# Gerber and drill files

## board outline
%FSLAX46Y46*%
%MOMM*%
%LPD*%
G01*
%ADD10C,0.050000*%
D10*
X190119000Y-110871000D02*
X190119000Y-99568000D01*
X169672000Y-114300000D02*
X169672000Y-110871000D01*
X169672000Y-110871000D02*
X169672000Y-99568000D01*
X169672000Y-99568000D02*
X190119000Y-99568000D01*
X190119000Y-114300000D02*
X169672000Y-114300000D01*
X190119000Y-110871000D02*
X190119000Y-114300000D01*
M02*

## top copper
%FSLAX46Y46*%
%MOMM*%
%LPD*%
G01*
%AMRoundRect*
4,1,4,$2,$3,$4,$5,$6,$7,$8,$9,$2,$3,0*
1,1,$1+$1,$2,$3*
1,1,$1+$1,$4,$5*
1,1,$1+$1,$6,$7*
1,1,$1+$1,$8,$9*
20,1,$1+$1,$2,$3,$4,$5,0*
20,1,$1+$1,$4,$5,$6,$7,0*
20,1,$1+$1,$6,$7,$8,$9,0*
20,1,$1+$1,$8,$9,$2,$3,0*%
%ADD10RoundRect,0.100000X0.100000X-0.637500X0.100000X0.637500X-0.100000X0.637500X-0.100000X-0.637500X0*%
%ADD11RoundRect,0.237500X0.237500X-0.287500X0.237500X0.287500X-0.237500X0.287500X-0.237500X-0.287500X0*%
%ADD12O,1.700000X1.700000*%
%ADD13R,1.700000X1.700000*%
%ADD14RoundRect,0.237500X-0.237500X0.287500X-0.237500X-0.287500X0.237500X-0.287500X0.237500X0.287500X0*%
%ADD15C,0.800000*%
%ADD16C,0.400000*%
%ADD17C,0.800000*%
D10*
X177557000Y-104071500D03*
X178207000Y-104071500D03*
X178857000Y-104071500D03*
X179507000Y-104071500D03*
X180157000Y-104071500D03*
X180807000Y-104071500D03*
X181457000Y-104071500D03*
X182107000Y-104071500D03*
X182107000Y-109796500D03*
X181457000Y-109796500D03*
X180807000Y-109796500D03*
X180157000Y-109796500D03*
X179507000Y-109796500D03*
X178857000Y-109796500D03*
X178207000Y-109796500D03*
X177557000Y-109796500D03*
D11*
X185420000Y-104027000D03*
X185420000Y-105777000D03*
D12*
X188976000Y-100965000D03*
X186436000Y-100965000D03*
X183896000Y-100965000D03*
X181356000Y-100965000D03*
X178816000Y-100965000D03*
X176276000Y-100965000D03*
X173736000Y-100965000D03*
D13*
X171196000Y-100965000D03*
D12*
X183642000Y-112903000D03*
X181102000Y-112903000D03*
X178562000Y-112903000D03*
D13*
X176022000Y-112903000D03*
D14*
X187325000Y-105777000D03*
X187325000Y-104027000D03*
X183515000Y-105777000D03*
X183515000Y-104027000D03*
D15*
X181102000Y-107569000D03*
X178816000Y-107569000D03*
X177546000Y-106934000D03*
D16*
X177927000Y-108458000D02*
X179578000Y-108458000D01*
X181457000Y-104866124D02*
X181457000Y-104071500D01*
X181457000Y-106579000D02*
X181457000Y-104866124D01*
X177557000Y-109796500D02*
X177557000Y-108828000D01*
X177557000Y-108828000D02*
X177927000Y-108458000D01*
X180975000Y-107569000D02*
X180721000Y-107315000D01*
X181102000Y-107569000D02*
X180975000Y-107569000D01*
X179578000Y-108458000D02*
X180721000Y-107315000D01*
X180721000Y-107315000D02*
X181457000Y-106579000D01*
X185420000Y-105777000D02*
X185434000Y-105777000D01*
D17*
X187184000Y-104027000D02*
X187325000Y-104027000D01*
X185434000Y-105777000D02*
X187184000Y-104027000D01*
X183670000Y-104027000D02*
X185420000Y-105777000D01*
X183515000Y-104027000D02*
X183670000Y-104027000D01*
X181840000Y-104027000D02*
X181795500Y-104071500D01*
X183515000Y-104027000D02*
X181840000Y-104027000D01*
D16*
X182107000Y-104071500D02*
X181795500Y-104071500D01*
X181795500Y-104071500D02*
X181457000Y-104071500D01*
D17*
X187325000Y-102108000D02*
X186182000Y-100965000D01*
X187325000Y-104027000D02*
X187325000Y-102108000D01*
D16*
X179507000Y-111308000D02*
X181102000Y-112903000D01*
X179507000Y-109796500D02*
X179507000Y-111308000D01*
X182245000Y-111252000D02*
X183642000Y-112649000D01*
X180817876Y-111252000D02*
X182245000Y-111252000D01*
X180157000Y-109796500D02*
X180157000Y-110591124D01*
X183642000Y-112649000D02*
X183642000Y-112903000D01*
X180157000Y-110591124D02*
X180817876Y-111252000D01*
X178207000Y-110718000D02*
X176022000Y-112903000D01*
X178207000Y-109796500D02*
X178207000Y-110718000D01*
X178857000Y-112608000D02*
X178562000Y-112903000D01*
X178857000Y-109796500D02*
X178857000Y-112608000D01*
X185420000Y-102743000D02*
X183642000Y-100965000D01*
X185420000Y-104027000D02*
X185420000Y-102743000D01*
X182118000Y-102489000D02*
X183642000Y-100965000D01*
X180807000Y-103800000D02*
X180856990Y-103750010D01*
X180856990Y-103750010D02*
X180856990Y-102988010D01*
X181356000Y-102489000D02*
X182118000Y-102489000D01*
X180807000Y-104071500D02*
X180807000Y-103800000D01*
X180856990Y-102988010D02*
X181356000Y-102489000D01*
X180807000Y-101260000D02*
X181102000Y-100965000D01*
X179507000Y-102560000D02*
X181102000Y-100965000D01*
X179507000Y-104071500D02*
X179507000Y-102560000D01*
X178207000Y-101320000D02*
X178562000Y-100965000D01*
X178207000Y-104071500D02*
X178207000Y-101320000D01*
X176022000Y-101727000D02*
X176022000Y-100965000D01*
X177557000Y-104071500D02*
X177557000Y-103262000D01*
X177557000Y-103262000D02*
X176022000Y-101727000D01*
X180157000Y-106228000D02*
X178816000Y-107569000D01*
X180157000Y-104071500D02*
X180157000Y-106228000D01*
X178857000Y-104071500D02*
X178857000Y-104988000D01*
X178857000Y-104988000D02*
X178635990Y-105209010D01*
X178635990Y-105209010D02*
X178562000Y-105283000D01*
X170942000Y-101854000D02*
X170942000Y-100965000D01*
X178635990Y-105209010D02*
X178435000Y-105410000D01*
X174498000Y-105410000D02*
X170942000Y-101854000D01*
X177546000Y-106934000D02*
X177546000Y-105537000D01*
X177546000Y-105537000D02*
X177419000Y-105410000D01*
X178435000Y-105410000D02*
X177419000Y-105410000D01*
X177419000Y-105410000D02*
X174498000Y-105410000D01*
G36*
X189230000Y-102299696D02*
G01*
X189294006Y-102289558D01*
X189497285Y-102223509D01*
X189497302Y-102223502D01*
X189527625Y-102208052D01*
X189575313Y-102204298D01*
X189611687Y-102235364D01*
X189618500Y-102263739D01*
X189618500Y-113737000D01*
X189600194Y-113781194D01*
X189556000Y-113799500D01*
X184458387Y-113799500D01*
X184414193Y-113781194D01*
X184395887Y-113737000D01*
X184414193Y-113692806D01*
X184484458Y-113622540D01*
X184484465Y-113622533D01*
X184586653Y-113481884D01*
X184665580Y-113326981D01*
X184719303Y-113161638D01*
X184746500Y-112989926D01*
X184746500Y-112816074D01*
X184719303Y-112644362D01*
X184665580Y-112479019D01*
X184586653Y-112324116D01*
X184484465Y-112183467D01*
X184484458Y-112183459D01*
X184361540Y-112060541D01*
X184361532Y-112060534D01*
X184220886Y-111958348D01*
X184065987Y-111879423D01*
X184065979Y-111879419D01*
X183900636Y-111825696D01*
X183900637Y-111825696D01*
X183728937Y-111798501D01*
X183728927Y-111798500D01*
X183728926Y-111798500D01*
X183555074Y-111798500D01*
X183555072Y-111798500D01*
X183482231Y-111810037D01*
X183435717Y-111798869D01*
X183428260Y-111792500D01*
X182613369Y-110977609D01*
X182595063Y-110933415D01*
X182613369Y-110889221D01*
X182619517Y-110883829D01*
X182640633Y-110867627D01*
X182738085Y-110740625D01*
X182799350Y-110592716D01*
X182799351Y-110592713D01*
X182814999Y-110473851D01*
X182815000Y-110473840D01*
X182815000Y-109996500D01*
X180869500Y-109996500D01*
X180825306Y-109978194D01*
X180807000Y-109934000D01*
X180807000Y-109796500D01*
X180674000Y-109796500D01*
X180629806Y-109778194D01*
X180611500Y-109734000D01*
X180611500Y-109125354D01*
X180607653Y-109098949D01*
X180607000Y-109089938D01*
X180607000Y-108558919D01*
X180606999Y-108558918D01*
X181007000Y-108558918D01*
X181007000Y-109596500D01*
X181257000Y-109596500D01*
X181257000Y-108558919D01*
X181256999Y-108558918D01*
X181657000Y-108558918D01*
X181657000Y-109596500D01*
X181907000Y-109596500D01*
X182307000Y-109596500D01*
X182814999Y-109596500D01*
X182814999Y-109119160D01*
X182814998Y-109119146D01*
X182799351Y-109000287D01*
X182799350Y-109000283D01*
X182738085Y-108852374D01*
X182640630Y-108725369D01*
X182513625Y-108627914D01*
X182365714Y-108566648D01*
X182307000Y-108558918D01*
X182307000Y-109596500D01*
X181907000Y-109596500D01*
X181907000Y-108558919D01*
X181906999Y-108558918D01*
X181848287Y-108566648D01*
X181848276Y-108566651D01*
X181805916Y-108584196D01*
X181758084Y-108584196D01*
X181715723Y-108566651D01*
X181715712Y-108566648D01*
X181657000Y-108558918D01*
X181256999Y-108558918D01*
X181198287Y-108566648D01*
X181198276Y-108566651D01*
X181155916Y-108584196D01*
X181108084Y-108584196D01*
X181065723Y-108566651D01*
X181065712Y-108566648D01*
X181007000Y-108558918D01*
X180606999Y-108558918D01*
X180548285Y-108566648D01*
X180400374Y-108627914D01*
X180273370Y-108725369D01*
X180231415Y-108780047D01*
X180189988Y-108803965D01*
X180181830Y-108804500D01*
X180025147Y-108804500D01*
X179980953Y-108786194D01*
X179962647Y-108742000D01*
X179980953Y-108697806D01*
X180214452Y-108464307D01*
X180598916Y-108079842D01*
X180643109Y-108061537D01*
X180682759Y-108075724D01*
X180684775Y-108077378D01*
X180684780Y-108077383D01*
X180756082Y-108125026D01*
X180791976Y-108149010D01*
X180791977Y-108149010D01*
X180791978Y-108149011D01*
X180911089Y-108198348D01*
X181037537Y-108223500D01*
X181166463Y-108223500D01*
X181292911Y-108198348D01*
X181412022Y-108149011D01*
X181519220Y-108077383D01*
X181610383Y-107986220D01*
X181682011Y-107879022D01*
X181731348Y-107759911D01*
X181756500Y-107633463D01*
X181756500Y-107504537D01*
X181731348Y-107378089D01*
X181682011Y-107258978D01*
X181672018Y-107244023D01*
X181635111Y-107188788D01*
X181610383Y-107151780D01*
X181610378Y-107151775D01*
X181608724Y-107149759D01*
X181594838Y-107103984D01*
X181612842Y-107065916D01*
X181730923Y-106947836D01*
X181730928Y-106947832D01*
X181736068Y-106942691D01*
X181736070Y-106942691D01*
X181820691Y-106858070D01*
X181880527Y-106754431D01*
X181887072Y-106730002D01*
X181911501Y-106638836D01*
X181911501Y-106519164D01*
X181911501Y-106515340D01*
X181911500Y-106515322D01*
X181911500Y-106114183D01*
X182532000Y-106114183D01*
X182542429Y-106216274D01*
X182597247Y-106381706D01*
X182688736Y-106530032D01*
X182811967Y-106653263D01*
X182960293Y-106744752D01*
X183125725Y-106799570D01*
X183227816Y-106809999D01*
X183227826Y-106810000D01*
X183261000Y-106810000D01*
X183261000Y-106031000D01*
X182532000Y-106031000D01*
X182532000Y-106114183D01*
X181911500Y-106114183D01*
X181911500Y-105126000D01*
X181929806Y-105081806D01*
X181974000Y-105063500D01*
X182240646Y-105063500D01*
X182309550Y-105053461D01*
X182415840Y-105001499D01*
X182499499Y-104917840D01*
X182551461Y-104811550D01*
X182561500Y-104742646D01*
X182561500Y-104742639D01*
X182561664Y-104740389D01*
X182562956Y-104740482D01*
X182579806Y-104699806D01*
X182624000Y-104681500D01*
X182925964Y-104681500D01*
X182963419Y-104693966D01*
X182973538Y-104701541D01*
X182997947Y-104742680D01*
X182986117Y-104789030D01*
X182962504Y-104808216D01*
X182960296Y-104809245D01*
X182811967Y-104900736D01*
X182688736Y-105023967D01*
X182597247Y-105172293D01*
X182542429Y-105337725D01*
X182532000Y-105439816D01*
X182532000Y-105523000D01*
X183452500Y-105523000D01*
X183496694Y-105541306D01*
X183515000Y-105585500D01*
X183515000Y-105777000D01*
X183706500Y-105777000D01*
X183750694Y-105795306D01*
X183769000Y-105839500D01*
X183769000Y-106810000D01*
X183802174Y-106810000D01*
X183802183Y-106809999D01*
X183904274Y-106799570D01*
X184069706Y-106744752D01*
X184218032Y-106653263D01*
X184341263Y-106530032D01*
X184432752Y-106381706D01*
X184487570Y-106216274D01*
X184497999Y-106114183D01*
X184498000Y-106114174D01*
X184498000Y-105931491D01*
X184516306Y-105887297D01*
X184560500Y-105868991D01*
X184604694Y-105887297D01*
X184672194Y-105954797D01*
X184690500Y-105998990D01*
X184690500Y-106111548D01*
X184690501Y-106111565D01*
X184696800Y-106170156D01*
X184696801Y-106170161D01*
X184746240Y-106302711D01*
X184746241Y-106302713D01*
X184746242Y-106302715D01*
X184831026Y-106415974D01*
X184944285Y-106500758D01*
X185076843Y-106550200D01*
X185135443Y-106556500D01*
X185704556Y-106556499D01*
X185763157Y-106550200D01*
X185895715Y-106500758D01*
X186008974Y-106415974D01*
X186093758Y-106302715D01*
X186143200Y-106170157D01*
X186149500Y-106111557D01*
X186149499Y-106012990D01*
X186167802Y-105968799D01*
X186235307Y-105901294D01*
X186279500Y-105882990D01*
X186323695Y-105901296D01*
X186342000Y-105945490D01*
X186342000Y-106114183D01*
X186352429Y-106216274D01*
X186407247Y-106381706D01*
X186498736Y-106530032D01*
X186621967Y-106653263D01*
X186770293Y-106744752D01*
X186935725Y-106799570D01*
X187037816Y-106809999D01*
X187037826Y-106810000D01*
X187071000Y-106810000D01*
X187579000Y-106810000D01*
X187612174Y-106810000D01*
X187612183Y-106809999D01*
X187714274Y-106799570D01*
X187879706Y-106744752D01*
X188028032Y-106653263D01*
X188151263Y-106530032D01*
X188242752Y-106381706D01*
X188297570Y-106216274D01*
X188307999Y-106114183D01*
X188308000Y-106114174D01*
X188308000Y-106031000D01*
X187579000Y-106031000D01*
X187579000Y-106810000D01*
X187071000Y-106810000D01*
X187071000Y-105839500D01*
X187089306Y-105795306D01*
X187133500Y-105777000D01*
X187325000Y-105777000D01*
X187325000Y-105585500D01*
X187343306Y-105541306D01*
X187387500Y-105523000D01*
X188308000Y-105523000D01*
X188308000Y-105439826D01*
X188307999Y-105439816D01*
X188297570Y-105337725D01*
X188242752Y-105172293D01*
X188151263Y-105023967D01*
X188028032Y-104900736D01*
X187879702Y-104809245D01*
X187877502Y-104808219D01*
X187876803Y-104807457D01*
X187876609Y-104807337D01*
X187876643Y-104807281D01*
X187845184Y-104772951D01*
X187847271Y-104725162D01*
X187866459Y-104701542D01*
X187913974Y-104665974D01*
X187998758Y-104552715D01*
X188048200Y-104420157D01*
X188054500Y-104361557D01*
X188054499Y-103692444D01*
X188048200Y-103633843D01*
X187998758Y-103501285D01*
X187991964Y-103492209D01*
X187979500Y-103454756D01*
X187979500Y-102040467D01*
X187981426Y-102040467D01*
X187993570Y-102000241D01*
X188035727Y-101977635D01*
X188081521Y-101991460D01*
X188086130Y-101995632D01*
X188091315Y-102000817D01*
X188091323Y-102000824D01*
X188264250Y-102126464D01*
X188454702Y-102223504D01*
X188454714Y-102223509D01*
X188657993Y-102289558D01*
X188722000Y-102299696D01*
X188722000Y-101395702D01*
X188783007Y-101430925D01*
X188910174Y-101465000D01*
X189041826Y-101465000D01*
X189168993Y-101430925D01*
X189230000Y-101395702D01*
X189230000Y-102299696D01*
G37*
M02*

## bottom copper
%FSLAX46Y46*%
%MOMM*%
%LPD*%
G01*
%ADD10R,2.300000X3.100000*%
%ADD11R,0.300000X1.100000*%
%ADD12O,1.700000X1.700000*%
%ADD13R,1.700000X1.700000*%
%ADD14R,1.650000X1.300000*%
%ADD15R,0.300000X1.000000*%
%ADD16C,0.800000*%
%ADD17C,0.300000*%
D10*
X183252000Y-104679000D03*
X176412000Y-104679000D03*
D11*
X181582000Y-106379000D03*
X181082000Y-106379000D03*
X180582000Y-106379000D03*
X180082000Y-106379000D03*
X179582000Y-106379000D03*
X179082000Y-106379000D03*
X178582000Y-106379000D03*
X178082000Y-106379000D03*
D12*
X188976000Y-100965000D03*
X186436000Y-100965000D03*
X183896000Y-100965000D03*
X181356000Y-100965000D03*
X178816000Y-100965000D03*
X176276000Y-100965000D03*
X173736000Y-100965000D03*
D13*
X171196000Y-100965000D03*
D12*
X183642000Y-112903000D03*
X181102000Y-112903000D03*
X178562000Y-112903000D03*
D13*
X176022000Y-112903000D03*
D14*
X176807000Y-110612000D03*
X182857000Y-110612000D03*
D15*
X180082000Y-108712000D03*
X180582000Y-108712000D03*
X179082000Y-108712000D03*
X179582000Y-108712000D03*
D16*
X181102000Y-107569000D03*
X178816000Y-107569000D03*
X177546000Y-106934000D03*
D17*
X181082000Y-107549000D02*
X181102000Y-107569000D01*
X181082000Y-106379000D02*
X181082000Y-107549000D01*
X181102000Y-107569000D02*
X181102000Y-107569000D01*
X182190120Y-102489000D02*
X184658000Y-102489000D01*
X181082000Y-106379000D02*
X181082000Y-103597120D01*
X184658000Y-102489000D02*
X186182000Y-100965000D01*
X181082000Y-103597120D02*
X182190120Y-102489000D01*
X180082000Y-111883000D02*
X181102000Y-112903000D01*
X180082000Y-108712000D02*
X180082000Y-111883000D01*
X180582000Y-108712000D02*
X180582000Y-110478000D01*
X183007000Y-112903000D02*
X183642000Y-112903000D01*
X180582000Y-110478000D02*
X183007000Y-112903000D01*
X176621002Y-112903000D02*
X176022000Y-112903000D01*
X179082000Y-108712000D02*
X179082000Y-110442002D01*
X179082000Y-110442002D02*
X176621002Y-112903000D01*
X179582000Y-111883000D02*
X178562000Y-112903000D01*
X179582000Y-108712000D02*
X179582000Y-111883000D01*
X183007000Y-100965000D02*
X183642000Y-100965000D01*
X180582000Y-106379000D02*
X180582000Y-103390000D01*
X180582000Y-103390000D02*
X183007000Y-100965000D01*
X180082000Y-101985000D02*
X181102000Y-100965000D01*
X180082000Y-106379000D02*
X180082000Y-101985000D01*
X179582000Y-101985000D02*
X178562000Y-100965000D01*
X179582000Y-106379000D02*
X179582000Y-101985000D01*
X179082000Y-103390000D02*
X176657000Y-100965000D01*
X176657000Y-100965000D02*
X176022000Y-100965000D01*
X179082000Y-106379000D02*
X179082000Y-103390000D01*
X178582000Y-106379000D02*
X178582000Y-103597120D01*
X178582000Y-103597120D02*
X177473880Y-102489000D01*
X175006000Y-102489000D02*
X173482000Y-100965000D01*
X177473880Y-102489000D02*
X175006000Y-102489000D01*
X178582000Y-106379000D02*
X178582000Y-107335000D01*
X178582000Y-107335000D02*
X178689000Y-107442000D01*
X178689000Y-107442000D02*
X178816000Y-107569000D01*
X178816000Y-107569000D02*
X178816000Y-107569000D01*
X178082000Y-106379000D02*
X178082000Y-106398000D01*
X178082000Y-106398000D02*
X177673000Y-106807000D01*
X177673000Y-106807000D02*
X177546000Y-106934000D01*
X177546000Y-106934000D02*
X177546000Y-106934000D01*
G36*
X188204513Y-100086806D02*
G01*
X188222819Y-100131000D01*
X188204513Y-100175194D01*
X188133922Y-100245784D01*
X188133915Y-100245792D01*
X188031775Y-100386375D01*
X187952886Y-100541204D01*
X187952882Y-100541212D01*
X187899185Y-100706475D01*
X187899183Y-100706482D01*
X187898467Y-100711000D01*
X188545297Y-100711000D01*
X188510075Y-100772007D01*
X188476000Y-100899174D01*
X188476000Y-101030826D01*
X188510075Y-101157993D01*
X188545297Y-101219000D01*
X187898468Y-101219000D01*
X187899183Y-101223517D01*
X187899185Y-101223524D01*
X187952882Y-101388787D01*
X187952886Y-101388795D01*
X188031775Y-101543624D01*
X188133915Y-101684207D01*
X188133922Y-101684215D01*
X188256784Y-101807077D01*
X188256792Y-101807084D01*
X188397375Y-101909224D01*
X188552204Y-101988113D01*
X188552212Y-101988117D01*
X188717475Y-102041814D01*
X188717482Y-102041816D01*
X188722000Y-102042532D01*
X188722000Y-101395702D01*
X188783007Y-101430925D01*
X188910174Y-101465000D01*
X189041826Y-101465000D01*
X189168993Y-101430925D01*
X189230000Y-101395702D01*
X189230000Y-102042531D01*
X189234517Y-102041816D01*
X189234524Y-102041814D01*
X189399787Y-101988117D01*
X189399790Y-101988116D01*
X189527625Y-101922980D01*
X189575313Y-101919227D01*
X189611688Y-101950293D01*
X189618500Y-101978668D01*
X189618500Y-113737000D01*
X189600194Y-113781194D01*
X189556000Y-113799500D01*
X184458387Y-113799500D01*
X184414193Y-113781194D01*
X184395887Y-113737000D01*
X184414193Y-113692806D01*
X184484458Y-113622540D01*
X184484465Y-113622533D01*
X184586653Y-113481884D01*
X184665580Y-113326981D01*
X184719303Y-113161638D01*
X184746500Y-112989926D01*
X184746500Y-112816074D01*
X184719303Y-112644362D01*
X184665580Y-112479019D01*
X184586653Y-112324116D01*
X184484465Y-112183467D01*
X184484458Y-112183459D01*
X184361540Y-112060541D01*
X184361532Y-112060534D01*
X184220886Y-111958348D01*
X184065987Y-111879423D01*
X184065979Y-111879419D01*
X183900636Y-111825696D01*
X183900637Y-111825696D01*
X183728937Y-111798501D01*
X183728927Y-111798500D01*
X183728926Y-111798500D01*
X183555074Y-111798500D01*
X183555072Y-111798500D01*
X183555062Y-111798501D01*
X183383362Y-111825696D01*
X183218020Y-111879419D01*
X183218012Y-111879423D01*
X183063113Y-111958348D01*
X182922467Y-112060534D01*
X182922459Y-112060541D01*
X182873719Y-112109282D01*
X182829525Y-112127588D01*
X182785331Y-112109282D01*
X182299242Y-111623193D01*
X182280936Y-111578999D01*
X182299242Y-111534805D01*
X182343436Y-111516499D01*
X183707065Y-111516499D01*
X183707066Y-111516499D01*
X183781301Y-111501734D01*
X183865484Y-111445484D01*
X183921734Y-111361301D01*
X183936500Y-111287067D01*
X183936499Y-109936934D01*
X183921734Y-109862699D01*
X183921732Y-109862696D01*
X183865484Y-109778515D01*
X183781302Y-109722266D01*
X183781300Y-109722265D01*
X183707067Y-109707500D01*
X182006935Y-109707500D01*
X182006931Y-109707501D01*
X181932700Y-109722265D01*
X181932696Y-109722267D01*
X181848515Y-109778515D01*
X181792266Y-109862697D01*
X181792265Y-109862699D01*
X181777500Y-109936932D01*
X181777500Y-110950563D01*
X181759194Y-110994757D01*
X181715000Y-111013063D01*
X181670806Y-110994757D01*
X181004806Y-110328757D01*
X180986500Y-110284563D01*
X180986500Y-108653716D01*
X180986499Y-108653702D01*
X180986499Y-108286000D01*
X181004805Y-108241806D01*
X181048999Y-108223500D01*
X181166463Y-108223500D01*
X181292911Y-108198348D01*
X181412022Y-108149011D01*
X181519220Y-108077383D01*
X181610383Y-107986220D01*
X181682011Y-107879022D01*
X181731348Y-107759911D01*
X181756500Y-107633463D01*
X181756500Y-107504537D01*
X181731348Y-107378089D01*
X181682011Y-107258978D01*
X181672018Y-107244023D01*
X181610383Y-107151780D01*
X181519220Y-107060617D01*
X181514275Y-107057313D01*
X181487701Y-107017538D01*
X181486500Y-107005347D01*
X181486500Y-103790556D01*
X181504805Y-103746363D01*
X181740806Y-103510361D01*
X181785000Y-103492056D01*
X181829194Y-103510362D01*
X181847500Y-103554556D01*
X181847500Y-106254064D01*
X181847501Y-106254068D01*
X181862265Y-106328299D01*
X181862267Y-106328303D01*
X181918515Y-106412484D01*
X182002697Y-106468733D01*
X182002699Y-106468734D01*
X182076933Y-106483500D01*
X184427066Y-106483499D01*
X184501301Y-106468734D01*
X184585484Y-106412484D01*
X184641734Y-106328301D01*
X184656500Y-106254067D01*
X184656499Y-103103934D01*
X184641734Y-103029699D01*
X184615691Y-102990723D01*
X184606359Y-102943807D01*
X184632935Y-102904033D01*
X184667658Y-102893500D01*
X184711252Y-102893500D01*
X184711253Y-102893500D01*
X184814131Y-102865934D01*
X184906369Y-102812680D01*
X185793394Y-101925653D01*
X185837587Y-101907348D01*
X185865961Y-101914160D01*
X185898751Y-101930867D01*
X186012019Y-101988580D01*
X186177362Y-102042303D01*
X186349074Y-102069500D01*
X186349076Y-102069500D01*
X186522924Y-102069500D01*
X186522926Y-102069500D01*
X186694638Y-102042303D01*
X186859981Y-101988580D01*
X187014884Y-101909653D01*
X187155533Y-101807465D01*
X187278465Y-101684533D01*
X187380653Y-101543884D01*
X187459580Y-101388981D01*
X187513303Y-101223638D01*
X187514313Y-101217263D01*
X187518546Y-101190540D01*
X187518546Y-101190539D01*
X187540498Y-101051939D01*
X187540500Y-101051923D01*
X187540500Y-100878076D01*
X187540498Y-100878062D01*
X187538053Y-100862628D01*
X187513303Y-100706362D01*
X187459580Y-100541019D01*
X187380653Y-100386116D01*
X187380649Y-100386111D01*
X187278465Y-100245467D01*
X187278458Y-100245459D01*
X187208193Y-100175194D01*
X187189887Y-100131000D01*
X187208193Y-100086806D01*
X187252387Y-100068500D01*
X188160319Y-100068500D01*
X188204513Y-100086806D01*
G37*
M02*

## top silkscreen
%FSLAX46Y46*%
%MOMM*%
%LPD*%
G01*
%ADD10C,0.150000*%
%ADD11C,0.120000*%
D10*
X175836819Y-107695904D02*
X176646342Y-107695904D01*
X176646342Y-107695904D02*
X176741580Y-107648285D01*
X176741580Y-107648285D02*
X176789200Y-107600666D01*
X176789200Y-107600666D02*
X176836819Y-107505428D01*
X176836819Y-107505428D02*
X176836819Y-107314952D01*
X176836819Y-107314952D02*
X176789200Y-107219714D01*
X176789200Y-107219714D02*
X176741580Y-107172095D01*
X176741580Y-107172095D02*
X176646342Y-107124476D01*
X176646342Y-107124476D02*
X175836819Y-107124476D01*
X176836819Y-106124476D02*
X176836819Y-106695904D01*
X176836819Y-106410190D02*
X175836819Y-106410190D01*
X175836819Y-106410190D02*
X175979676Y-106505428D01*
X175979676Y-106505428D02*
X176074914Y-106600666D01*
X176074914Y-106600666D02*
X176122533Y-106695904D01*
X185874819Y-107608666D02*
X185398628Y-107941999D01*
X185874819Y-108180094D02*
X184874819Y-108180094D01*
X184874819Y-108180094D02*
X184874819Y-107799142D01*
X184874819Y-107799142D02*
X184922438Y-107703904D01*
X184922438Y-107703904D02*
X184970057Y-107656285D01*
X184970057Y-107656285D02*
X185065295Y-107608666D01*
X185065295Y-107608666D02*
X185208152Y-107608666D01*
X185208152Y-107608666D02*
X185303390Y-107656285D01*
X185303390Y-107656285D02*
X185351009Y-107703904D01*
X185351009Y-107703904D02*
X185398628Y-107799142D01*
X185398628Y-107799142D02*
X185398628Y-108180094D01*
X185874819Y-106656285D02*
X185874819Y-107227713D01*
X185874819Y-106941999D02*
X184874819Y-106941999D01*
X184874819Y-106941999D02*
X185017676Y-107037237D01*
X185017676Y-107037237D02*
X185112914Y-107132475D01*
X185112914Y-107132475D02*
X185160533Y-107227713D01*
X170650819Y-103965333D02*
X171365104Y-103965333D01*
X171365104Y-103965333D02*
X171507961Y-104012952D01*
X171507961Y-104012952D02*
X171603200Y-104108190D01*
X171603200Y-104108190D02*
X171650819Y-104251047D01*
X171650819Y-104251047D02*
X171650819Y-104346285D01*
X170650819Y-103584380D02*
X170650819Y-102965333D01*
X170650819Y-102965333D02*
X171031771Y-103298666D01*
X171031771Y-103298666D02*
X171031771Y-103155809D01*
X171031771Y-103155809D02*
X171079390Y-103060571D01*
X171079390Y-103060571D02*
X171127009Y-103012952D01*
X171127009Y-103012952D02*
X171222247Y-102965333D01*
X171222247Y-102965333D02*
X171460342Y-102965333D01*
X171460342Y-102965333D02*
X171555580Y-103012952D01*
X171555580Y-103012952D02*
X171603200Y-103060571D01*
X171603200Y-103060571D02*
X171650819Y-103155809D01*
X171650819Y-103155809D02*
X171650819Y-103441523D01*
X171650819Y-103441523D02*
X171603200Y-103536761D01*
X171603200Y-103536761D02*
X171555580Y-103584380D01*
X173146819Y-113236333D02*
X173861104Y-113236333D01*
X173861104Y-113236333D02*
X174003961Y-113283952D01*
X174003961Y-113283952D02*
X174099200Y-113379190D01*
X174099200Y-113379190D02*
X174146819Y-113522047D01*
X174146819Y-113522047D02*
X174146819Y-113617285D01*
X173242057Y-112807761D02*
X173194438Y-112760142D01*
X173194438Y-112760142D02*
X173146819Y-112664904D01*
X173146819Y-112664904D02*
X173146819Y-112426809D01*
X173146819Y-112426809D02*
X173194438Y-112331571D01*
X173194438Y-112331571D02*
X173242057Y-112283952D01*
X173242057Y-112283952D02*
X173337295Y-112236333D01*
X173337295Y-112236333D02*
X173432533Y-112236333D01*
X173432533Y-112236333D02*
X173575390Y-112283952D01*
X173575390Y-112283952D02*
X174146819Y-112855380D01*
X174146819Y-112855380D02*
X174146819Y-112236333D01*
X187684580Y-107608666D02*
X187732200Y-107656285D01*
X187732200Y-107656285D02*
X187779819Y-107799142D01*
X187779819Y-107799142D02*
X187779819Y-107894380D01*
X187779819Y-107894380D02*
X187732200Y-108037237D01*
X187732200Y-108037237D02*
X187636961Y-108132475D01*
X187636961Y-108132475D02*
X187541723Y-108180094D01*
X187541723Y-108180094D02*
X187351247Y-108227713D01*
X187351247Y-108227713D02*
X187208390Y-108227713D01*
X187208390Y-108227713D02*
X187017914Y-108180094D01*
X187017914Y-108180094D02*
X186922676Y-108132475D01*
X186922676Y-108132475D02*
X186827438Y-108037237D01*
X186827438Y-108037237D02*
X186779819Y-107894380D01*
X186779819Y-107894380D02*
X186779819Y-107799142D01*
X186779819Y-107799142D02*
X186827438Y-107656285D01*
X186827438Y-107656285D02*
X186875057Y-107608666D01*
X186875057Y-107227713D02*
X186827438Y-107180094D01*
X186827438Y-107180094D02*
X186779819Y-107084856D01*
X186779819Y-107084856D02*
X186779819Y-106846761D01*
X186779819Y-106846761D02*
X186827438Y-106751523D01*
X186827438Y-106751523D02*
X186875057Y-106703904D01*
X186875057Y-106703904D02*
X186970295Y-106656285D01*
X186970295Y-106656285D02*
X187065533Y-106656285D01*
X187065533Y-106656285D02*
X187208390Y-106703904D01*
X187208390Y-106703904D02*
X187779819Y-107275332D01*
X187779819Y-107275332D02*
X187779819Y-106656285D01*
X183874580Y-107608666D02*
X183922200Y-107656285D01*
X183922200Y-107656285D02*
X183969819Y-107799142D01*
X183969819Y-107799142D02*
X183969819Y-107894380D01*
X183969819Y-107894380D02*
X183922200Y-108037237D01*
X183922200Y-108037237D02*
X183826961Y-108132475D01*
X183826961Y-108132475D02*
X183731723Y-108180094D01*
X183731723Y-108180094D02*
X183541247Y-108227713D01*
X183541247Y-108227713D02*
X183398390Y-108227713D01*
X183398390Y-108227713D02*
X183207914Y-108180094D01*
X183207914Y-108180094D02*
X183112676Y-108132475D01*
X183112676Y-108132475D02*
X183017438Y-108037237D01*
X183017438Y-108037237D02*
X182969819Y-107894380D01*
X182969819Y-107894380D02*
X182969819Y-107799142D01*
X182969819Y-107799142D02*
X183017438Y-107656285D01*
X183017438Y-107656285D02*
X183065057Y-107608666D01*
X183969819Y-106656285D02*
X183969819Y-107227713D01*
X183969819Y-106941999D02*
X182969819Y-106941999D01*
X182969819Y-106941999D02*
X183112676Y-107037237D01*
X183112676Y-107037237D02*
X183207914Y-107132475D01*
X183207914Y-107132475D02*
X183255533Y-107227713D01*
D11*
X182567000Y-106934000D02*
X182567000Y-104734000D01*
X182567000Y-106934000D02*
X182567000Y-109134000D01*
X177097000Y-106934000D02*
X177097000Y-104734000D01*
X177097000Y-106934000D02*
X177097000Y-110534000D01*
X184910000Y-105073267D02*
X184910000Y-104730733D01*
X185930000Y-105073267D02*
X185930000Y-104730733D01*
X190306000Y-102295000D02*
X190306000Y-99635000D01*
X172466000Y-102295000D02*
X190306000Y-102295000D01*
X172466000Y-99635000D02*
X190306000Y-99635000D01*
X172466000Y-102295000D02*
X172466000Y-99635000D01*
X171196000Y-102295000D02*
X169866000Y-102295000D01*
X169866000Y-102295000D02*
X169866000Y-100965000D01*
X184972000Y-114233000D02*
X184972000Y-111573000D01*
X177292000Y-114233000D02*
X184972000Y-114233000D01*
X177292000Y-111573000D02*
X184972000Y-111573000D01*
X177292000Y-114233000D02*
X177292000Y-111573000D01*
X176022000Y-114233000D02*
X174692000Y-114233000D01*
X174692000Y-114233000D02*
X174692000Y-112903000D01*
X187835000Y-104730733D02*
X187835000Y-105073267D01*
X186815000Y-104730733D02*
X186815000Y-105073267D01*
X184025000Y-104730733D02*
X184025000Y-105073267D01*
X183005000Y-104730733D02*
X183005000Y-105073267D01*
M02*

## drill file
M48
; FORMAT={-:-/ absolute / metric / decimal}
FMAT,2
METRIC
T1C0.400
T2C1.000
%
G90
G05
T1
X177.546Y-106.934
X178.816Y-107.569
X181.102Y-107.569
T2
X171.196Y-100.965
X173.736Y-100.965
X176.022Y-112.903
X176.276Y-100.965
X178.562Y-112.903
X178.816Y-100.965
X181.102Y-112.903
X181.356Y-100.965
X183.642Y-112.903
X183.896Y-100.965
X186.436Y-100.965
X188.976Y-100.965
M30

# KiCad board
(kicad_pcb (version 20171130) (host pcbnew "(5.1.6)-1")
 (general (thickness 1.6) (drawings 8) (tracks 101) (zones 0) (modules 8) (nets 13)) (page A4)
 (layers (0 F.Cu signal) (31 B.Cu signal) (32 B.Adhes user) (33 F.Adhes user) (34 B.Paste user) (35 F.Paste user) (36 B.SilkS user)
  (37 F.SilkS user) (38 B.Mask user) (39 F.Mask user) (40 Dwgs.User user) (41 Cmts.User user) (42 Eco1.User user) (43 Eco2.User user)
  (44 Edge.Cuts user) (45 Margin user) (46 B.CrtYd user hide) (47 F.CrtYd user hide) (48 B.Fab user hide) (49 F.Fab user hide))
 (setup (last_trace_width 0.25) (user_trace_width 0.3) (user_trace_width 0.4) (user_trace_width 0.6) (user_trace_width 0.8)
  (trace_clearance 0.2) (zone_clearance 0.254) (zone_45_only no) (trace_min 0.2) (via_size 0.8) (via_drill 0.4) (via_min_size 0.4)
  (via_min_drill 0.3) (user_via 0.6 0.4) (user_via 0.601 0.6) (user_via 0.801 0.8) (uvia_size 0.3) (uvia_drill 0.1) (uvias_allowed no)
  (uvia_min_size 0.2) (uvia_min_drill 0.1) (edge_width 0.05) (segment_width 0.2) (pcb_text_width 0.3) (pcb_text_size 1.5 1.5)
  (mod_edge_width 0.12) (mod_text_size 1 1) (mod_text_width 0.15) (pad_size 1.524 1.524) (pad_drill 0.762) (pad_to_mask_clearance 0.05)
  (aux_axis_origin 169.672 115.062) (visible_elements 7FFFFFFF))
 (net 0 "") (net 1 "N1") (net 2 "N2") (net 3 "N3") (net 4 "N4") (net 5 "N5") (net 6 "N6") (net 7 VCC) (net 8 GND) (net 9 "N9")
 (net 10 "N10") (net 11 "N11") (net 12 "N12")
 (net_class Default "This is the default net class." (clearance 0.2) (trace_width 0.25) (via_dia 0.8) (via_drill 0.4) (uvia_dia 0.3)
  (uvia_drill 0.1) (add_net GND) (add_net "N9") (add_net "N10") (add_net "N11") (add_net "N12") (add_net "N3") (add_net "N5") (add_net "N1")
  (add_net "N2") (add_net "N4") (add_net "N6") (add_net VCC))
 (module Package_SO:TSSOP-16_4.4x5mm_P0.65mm (layer F.Cu) (at 179.832 106.934 90)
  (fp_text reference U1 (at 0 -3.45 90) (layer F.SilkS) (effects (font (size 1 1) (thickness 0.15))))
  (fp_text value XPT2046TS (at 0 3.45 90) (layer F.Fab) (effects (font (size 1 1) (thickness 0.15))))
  (fp_line (start 0 2.735) (end 2.2 2.735) (layer F.SilkS) (width 0.12))
  (fp_line (start 0 2.735) (end -2.2 2.735) (layer F.SilkS) (width 0.12))
  (fp_line (start 0 -2.735) (end 2.2 -2.735) (layer F.SilkS) (width 0.12))
  (fp_line (start 0 -2.735) (end -3.6 -2.735) (layer F.SilkS) (width 0.12))
  (pad 16 smd roundrect (at 2.8625 -2.275 90) (size 1.475 0.4) (layers F.Cu F.Paste F.Mask) (roundrect_rratio 0.25) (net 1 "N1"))
  (pad 15 smd roundrect (at 2.8625 -1.625 90) (size 1.475 0.4) (layers F.Cu F.Paste F.Mask) (roundrect_rratio 0.25) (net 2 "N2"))
  (pad 14 smd roundrect (at 2.8625 -0.975 90) (size 1.475 0.4) (layers F.Cu F.Paste F.Mask) (roundrect_rratio 0.25) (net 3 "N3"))
  (pad 13 smd roundrect (at 2.8625 -0.325 90) (size 1.475 0.4) (layers F.Cu F.Paste F.Mask) (roundrect_rratio 0.25) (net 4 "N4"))
  (pad 12 smd roundrect (at 2.8625 0.325 90) (size 1.475 0.4) (layers F.Cu F.Paste F.Mask) (roundrect_rratio 0.25) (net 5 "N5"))
  (pad 11 smd roundrect (at 2.8625 0.975 90) (size 1.475 0.4) (layers F.Cu F.Paste F.Mask) (roundrect_rratio 0.25) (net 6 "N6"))
  (pad 10 smd roundrect (at 2.8625 1.625 90) (size 1.475 0.4) (layers F.Cu F.Paste F.Mask) (roundrect_rratio 0.25) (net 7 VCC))
  (pad 9 smd roundrect (at 2.8625 2.275 90) (size 1.475 0.4) (layers F.Cu F.Paste F.Mask) (roundrect_rratio 0.25) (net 7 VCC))
  (pad 8 smd roundrect (at -2.8625 2.275 90) (size 1.475 0.4) (layers F.Cu F.Paste F.Mask) (roundrect_rratio 0.25) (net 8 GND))
  (pad 7 smd roundrect (at -2.8625 1.625 90) (size 1.475 0.4) (layers F.Cu F.Paste F.Mask) (roundrect_rratio 0.25) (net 8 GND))
  (pad 6 smd roundrect (at -2.8625 0.975 90) (size 1.475 0.4) (layers F.Cu F.Paste F.Mask) (roundrect_rratio 0.25) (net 8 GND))
  (pad 5 smd roundrect (at -2.8625 0.325 90) (size 1.475 0.4) (layers F.Cu F.Paste F.Mask) (roundrect_rratio 0.25) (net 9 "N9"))
  (pad 4 smd roundrect (at -2.8625 -0.325 90) (size 1.475 0.4) (layers F.Cu F.Paste F.Mask) (roundrect_rratio 0.25) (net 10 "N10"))
  (pad 3 smd roundrect (at -2.8625 -0.975 90) (size 1.475 0.4) (layers F.Cu F.Paste F.Mask) (roundrect_rratio 0.25) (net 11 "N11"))
  (pad 2 smd roundrect (at -2.8625 -1.625 90) (size 1.475 0.4) (layers F.Cu F.Paste F.Mask) (roundrect_rratio 0.25) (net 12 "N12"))
  (pad 1 smd roundrect (at -2.8625 -2.275 90) (size 1.475 0.4) (layers F.Cu F.Paste F.Mask) (roundrect_rratio 0.25) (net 7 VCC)))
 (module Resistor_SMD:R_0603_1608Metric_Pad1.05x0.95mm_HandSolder (layer F.Cu) (at 185.42 104.902 90)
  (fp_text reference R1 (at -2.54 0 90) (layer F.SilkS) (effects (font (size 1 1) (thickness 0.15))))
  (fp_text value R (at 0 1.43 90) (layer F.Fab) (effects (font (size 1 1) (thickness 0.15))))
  (fp_line (start -0.171267 -0.51) (end 0.171267 -0.51) (layer F.SilkS) (width 0.12))
  (fp_line (start -0.171267 0.51) (end 0.171267 0.51) (layer F.SilkS) (width 0.12))
  (pad 2 smd roundrect (at 0.875 0 90) (size 1.05 0.95) (layers F.Cu F.Paste F.Mask) (roundrect_rratio 0.25) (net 6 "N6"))
  (pad 1 smd roundrect (at -0.875 0 90) (size 1.05 0.95) (layers F.Cu F.Paste F.Mask) (roundrect_rratio 0.25) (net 7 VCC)))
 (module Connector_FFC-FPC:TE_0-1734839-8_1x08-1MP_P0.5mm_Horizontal (layer B.Cu) (at 179.832 105.029)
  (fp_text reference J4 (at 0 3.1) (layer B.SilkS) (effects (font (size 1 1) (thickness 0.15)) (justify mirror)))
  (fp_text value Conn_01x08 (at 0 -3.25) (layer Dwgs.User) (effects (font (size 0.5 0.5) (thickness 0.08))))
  (pad MP smd rect (at 3.42 -0.35) (size 2.3 3.1) (layers B.Cu B.Paste B.Mask))
  (pad MP smd rect (at -3.42 -0.35) (size 2.3 3.1) (layers B.Cu B.Paste B.Mask))
  (pad 8 smd rect (at 1.75 1.35) (size 0.3 1.1) (layers B.Cu B.Paste B.Mask) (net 8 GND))
  (pad 7 smd rect (at 1.25 1.35) (size 0.3 1.1) (layers B.Cu B.Paste B.Mask) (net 7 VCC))
  (pad 6 smd rect (at 0.75 1.35) (size 0.3 1.1) (layers B.Cu B.Paste B.Mask) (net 6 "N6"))
  (pad 5 smd rect (at 0.25 1.35) (size 0.3 1.1) (layers B.Cu B.Paste B.Mask) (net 4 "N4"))
  (pad 4 smd rect (at -0.25 1.35) (size 0.3 1.1) (layers B.Cu B.Paste B.Mask) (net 2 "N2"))
  (pad 3 smd rect (at -0.75 1.35) (size 0.3 1.1) (layers B.Cu B.Paste B.Mask) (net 1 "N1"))
  (pad 2 smd rect (at -1.25 1.35) (size 0.3 1.1) (layers B.Cu B.Paste B.Mask) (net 5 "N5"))
  (pad 1 smd rect (at -1.75 1.35) (size 0.3 1.1) (layers B.Cu B.Paste B.Mask) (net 3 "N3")))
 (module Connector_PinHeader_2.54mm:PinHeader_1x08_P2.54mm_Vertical (layer F.Cu) (at 171.196 100.965 90)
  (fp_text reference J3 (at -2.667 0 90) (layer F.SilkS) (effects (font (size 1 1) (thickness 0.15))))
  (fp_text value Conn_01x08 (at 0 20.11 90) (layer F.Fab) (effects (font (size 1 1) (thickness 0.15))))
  (fp_line (start -1.33 19.11) (end 1.33 19.11) (layer F.SilkS) (width 0.12))
  (fp_line (start -1.33 1.27) (end -1.33 19.11) (layer F.SilkS) (width 0.12))
  (fp_line (start 1.33 1.27) (end 1.33 19.11) (layer F.SilkS) (width 0.12))
  (fp_line (start -1.33 1.27) (end 1.33 1.27) (layer F.SilkS) (width 0.12))
  (fp_line (start -1.33 0) (end -1.33 -1.33) (layer F.SilkS) (width 0.12))
  (fp_line (start -1.33 -1.33) (end 0 -1.33) (layer F.SilkS) (width 0.12))
  (pad 8 thru_hole oval (at 0 17.78 90) (size 1.7 1.7) (drill 1) (layers *.Cu *.Mask) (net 8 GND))
  (pad 7 thru_hole oval (at 0 15.24 90) (size 1.7 1.7) (drill 1) (layers *.Cu *.Mask) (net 7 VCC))
  (pad 6 thru_hole oval (at 0 12.7 90) (size 1.7 1.7) (drill 1) (layers *.Cu *.Mask) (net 6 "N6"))
  (pad 5 thru_hole oval (at 0 10.16 90) (size 1.7 1.7) (drill 1) (layers *.Cu *.Mask) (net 4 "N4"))
  (pad 4 thru_hole oval (at 0 7.62 90) (size 1.7 1.7) (drill 1) (layers *.Cu *.Mask) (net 2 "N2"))
  (pad 3 thru_hole oval (at 0 5.08 90) (size 1.7 1.7) (drill 1) (layers *.Cu *.Mask) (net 1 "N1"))
  (pad 2 thru_hole oval (at 0 2.54 90) (size 1.7 1.7) (drill 1) (layers *.Cu *.Mask) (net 5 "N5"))
  (pad 1 thru_hole rect (at 0 0 90) (size 1.7 1.7) (drill 1) (layers *.Cu *.Mask) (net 3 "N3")))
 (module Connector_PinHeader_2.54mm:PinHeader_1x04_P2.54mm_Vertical (layer F.Cu) (at 176.022 112.903 90)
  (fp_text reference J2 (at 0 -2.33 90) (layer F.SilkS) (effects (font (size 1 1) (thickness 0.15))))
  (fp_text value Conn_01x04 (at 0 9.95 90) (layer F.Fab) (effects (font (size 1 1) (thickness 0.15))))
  (fp_line (start -1.33 8.95) (end 1.33 8.95) (layer F.SilkS) (width 0.12))
  (fp_line (start -1.33 1.27) (end -1.33 8.95) (layer F.SilkS) (width 0.12))
  (fp_line (start 1.33 1.27) (end 1.33 8.95) (layer F.SilkS) (width 0.12))
  (fp_line (start -1.33 1.27) (end 1.33 1.27) (layer F.SilkS) (width 0.12))
  (fp_line (start -1.33 0) (end -1.33 -1.33) (layer F.SilkS) (width 0.12))
  (fp_line (start -1.33 -1.33) (end 0 -1.33) (layer F.SilkS) (width 0.12))
  (pad 4 thru_hole oval (at 0 7.62 90) (size 1.7 1.7) (drill 1) (layers *.Cu *.Mask) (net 9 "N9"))
  (pad 3 thru_hole oval (at 0 5.08 90) (size 1.7 1.7) (drill 1) (layers *.Cu *.Mask) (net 10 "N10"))
  (pad 2 thru_hole oval (at 0 2.54 90) (size 1.7 1.7) (drill 1) (layers *.Cu *.Mask) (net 11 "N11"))
  (pad 1 thru_hole rect (at 0 0 90) (size 1.7 1.7) (drill 1) (layers *.Cu *.Mask) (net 12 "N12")))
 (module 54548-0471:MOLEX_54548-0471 (layer B.Cu) (at 179.832 108.712 180)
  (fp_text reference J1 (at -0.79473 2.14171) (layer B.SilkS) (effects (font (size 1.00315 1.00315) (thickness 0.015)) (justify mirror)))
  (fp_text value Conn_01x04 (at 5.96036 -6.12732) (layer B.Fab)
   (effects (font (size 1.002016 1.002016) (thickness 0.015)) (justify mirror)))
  (pad S2 smd rect (at 3.025 -1.9 180) (size 1.65 1.3) (layers B.Cu B.Paste B.Mask))
  (pad S1 smd rect (at -3.025 -1.9 180) (size 1.65 1.3) (layers B.Cu B.Paste B.Mask))
  (pad 2 smd rect (at -0.25 0 180) (size 0.3 1) (layers B.Cu B.Paste B.Mask) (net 10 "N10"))
  (pad 1 smd rect (at -0.75 0 180) (size 0.3 1) (layers B.Cu B.Paste B.Mask) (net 9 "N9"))
  (pad 4 smd rect (at 0.75 0 180) (size 0.3 1) (layers B.Cu B.Paste B.Mask) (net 12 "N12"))
  (pad 3 smd rect (at 0.25 0 180) (size 0.3 1) (layers B.Cu B.Paste B.Mask) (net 11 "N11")))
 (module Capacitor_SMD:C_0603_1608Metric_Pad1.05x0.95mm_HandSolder (layer F.Cu) (at 187.325 104.902 270)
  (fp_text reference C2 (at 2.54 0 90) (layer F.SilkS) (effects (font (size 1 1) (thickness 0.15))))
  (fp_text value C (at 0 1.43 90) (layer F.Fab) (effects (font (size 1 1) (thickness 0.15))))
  (fp_line (start -0.171267 -0.51) (end 0.171267 -0.51) (layer F.SilkS) (width 0.12))
  (fp_line (start -0.171267 0.51) (end 0.171267 0.51) (layer F.SilkS) (width 0.12))
  (pad 2 smd roundrect (at 0.875 0 270) (size 1.05 0.95) (layers F.Cu F.Paste F.Mask) (roundrect_rratio 0.25) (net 8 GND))
  (pad 1 smd roundrect (at -0.875 0 270) (size 1.05 0.95) (layers F.Cu F.Paste F.Mask) (roundrect_rratio 0.25) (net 7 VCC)))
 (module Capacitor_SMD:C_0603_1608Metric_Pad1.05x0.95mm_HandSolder (layer F.Cu) (at 183.515 104.902 270)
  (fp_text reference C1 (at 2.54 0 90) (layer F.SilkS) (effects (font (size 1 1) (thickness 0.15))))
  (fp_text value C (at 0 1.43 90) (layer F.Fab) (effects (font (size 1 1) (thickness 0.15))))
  (fp_line (start -0.171267 -0.51) (end 0.171267 -0.51) (layer F.SilkS) (width 0.12))
  (fp_line (start -0.171267 0.51) (end 0.171267 0.51) (layer F.SilkS) (width 0.12))
  (pad 2 smd roundrect (at 0.875 0 270) (size 1.05 0.95) (layers F.Cu F.Paste F.Mask) (roundrect_rratio 0.25) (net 8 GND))
  (pad 1 smd roundrect (at -0.875 0 270) (size 1.05 0.95) (layers F.Cu F.Paste F.Mask) (roundrect_rratio 0.25) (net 7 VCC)))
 (gr_line (start 190.119 110.871) (end 190.119 99.568) (layer Edge.Cuts) (width 0.05))
 (gr_line (start 169.672 114.3) (end 169.672 110.871) (layer Edge.Cuts) (width 0.05))
 (gr_line (start 169.672 110.871) (end 169.672 99.568) (layer Edge.Cuts) (width 0.05))
 (gr_line (start 169.672 99.568) (end 190.119 99.568) (layer Edge.Cuts) (width 0.05))
 (gr_line (start 190.119 114.3) (end 169.672 114.3) (layer Edge.Cuts) (width 0.05))
 (gr_line (start 190.119 110.871) (end 190.119 114.3) (layer Edge.Cuts) (width 0.05))
 (segment (start 177.927 108.458) (end 179.578 108.458) (width 0.4) (layer F.Cu) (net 7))
 (segment (start 181.457 104.866124) (end 181.457 104.0715) (width 0.4) (layer F.Cu) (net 7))
 (segment (start 181.457 106.579) (end 181.457 104.866124) (width 0.4) (layer F.Cu) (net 7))
 (segment (start 177.557 109.7965) (end 177.557 108.828) (width 0.4) (layer F.Cu) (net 7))
 (segment (start 177.557 108.828) (end 177.927 108.458) (width 0.4) (layer F.Cu) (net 7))
 (segment (start 181.082 107.549) (end 181.102 107.569) (width 0.3) (layer B.Cu) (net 7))
 (segment (start 181.082 106.379) (end 181.082 107.549) (width 0.3) (layer B.Cu) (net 7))
 (segment (start 181.102 107.569) (end 181.102 107.569) (width 0.3) (layer B.Cu) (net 7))
 (via (at 181.102 107.569) (size 0.8) (drill 0.4) (layers F.Cu B.Cu) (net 7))
 (segment (start 180.975 107.569) (end 180.721 107.315) (width 0.4) (layer F.Cu) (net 7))
 (segment (start 181.102 107.569) (end 180.975 107.569) (width 0.4) (layer F.Cu) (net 7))
 (segment (start 179.578 108.458) (end 180.721 107.315) (width 0.4) (layer F.Cu) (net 7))
 (segment (start 180.721 107.315) (end 181.457 106.579) (width 0.4) (layer F.Cu) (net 7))
 (segment (start 185.42 105.777) (end 185.434 105.777) (width 0.4) (layer F.Cu) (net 7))
 (segment (start 187.184 104.027) (end 187.325 104.027) (width 0.8) (layer F.Cu) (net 7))
 (segment (start 185.434 105.777) (end 187.184 104.027) (width 0.8) (layer F.Cu) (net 7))
 (segment (start 183.67 104.027) (end 185.42 105.777) (width 0.8) (layer F.Cu) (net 7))
 (segment (start 183.515 104.027) (end 183.67 104.027) (width 0.8) (layer F.Cu) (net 7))
 (segment (start 181.84 104.027) (end 181.7955 104.0715) (width 0.8) (layer F.Cu) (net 7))
 (segment (start 183.515 104.027) (end 181.84 104.027) (width 0.8) (layer F.Cu) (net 7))
 (segment (start 182.107 104.0715) (end 181.7955 104.0715) (width 0.4) (layer F.Cu) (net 7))
 (segment (start 181.7955 104.0715) (end 181.457 104.0715) (width 0.4) (layer F.Cu) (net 7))
 (segment (start 187.325 102.108) (end 186.182 100.965) (width 0.8) (layer F.Cu) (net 7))
 (segment (start 187.325 104.027) (end 187.325 102.108) (width 0.8) (layer F.Cu) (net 7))
 (segment (start 182.19012 102.489) (end 184.658 102.489) (width 0.3) (layer B.Cu) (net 7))
 (segment (start 181.082 106.379) (end 181.082 103.59712) (width 0.3) (layer B.Cu) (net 7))
 (segment (start 184.658 102.489) (end 186.182 100.965) (width 0.3) (layer B.Cu) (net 7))
 (segment (start 181.082 103.59712) (end 182.19012 102.489) (width 0.3) (layer B.Cu) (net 7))
 (segment (start 179.507 111.308) (end 181.102 112.903) (width 0.4) (layer F.Cu) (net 10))
 (segment (start 179.507 109.7965) (end 179.507 111.308) (width 0.4) (layer F.Cu) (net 10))
 (segment (start 180.082 111.883) (end 181.102 112.903) (width 0.3) (layer B.Cu) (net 10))
 (segment (start 180.082 108.712) (end 180.082 111.883) (width 0.3) (layer B.Cu) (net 10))
 (segment (start 182.245 111.252) (end 183.642 112.649) (width 0.4) (layer F.Cu) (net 9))
 (segment (start 180.817876 111.252) (end 182.245 111.252) (width 0.4) (layer F.Cu) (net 9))
 (segment (start 180.157 109.7965) (end 180.157 110.591124) (width 0.4) (layer F.Cu) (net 9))
 (segment (start 183.642 112.649) (end 183.642 112.903) (width 0.4) (layer F.Cu) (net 9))
 (segment (start 180.157 110.591124) (end 180.817876 111.252) (width 0.4) (layer F.Cu) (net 9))
 (segment (start 180.582 108.712) (end 180.582 110.478) (width 0.3) (layer B.Cu) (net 9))
 (segment (start 183.007 112.903) (end 183.642 112.903) (width 0.3) (layer B.Cu) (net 9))
 (segment (start 180.582 110.478) (end 183.007 112.903) (width 0.3) (layer B.Cu) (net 9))
 (segment (start 178.207 110.718) (end 176.022 112.903) (width 0.4) (layer F.Cu) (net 12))
 (segment (start 178.207 109.7965) (end 178.207 110.718) (width 0.4) (layer F.Cu) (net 12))
 (segment (start 176.621002 112.903) (end 176.022 112.903) (width 0.3) (layer B.Cu) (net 12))
 (segment (start 179.082 108.712) (end 179.082 110.442002) (width 0.3) (layer B.Cu) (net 12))
 (segment (start 179.082 110.442002) (end 176.621002 112.903) (width 0.3) (layer B.Cu) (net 12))
 (segment (start 178.857 112.608) (end 178.562 112.903) (width 0.4) (layer F.Cu) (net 11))
 (segment (start 178.857 109.7965) (end 178.857 112.608) (width 0.4) (layer F.Cu) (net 11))
 (segment (start 179.582 111.883) (end 178.562 112.903) (width 0.3) (layer B.Cu) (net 11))
 (segment (start 179.582 108.712) (end 179.582 111.883) (width 0.3) (layer B.Cu) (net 11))
 (segment (start 185.42 102.743) (end 183.642 100.965) (width 0.4) (layer F.Cu) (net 6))
 (segment (start 185.42 104.027) (end 185.42 102.743) (width 0.4) (layer F.Cu) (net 6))
 (segment (start 182.118 102.489) (end 183.642 100.965) (width 0.4) (layer F.Cu) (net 6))
 (segment (start 180.807 103.8) (end 180.85699 103.75001) (width 0.4) (layer F.Cu) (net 6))
 (segment (start 180.85699 103.75001) (end 180.85699 102.98801) (width 0.4) (layer F.Cu) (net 6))
 (segment (start 181.356 102.489) (end 182.118 102.489) (width 0.4) (layer F.Cu) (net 6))
 (segment (start 180.807 104.0715) (end 180.807 103.8) (width 0.4) (layer F.Cu) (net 6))
 (segment (start 180.85699 102.98801) (end 181.356 102.489) (width 0.4) (layer F.Cu) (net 6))
 (segment (start 183.007 100.965) (end 183.642 100.965) (width 0.3) (layer B.Cu) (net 6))
 (segment (start 180.582 106.379) (end 180.582 103.39) (width 0.3) (layer B.Cu) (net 6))
 (segment (start 180.582 103.39) (end 183.007 100.965) (width 0.3) (layer B.Cu) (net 6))
 (segment (start 180.807 101.26) (end 181.102 100.965) (width 0.4) (layer F.Cu) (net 4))
 (segment (start 180.082 101.985) (end 181.102 100.965) (width 0.3) (layer B.Cu) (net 4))
 (segment (start 180.082 106.379) (end 180.082 101.985) (width 0.3) (layer B.Cu) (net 4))
 (segment (start 179.507 102.56) (end 181.102 100.965) (width 0.4) (layer F.Cu) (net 4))
 (segment (start 179.507 104.0715) (end 179.507 102.56) (width 0.4) (layer F.Cu) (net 4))
 (segment (start 178.207 101.32) (end 178.562 100.965) (width 0.4) (layer F.Cu) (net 2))
 (segment (start 178.207 104.0715) (end 178.207 101.32) (width 0.4) (layer F.Cu) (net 2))
 (segment (start 179.582 101.985) (end 178.562 100.965) (width 0.3) (layer B.Cu) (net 2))
 (segment (start 179.582 106.379) (end 179.582 101.985) (width 0.3) (layer B.Cu) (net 2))
 (segment (start 179.082 103.39) (end 176.657 100.965) (width 0.3) (layer B.Cu) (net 1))
 (segment (start 176.657 100.965) (end 176.022 100.965) (width 0.3) (layer B.Cu) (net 1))
 (segment (start 179.082 106.379) (end 179.082 103.39) (width 0.3) (layer B.Cu) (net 1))
 (segment (start 176.022 101.727) (end 176.022 100.965) (width 0.4) (layer F.Cu) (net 1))
 (segment (start 177.557 104.0715) (end 177.557 103.262) (width 0.4) (layer F.Cu) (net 1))
 (segment (start 177.557 103.262) (end 176.022 101.727) (width 0.4) (layer F.Cu) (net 1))
 (segment (start 178.582 106.379) (end 178.582 103.59712) (width 0.3) (layer B.Cu) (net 5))
 (segment (start 178.582 103.59712) (end 177.47388 102.489) (width 0.3) (layer B.Cu) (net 5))
 (segment (start 175.006 102.489) (end 173.482 100.965) (width 0.3) (layer B.Cu) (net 5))
 (segment (start 177.47388 102.489) (end 175.006 102.489) (width 0.3) (layer B.Cu) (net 5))
 (segment (start 178.582 106.379) (end 178.582 107.335) (width 0.3) (layer B.Cu) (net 5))
 (segment (start 178.582 107.335) (end 178.689 107.442) (width 0.3) (layer B.Cu) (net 5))
 (segment (start 178.689 107.442) (end 178.816 107.569) (width 0.3) (layer B.Cu) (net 5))
 (segment (start 178.816 107.569) (end 178.816 107.569) (width 0.3) (layer B.Cu) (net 5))
 (via (at 178.816 107.569) (size 0.8) (drill 0.4) (layers F.Cu B.Cu) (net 5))
 (segment (start 180.157 106.228) (end 178.816 107.569) (width 0.4) (layer F.Cu) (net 5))
 (segment (start 180.157 104.0715) (end 180.157 106.228) (width 0.4) (layer F.Cu) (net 5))
 (segment (start 178.857 104.0715) (end 178.857 104.988) (width 0.4) (layer F.Cu) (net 3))
 (segment (start 178.857 104.988) (end 178.63599 105.20901) (width 0.4) (layer F.Cu) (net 3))
 (segment (start 178.63599 105.20901) (end 178.562 105.283) (width 0.4) (layer F.Cu) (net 3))
 (segment (start 170.942 101.854) (end 170.942 100.965) (width 0.4) (layer F.Cu) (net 3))
 (segment (start 178.63599 105.20901) (end 178.435 105.41) (width 0.4) (layer F.Cu) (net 3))
 (segment (start 174.498 105.41) (end 170.942 101.854) (width 0.4) (layer F.Cu) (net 3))
 (segment (start 178.082 106.379) (end 178.082 106.398) (width 0.3) (layer B.Cu) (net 3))
 (segment (start 178.082 106.398) (end 177.673 106.807) (width 0.3) (layer B.Cu) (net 3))
 (segment (start 177.673 106.807) (end 177.546 106.934) (width 0.3) (layer B.Cu) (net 3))
 (segment (start 177.546 106.934) (end 177.546 106.934) (width 0.3) (layer B.Cu) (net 3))
 (via (at 177.546 106.934) (size 0.8) (drill 0.4) (layers F.Cu B.Cu) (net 3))
 (segment (start 177.546 106.934) (end 177.546 105.537) (width 0.4) (layer F.Cu) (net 3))
 (segment (start 177.546 105.537) (end 177.419 105.41) (width 0.4) (layer F.Cu) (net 3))
 (segment (start 178.435 105.41) (end 177.419 105.41) (width 0.4) (layer F.Cu) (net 3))
 (segment (start 177.419 105.41) (end 174.498 105.41) (width 0.4) (layer F.Cu) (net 3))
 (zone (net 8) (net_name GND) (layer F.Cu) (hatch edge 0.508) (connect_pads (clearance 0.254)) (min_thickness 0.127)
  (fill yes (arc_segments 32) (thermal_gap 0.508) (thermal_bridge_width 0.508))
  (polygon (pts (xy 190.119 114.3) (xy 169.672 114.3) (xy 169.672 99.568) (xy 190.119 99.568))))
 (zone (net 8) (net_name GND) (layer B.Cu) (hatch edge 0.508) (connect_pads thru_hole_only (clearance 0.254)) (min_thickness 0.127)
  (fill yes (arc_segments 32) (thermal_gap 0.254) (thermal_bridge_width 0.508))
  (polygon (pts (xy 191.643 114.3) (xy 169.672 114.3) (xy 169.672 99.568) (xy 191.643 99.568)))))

